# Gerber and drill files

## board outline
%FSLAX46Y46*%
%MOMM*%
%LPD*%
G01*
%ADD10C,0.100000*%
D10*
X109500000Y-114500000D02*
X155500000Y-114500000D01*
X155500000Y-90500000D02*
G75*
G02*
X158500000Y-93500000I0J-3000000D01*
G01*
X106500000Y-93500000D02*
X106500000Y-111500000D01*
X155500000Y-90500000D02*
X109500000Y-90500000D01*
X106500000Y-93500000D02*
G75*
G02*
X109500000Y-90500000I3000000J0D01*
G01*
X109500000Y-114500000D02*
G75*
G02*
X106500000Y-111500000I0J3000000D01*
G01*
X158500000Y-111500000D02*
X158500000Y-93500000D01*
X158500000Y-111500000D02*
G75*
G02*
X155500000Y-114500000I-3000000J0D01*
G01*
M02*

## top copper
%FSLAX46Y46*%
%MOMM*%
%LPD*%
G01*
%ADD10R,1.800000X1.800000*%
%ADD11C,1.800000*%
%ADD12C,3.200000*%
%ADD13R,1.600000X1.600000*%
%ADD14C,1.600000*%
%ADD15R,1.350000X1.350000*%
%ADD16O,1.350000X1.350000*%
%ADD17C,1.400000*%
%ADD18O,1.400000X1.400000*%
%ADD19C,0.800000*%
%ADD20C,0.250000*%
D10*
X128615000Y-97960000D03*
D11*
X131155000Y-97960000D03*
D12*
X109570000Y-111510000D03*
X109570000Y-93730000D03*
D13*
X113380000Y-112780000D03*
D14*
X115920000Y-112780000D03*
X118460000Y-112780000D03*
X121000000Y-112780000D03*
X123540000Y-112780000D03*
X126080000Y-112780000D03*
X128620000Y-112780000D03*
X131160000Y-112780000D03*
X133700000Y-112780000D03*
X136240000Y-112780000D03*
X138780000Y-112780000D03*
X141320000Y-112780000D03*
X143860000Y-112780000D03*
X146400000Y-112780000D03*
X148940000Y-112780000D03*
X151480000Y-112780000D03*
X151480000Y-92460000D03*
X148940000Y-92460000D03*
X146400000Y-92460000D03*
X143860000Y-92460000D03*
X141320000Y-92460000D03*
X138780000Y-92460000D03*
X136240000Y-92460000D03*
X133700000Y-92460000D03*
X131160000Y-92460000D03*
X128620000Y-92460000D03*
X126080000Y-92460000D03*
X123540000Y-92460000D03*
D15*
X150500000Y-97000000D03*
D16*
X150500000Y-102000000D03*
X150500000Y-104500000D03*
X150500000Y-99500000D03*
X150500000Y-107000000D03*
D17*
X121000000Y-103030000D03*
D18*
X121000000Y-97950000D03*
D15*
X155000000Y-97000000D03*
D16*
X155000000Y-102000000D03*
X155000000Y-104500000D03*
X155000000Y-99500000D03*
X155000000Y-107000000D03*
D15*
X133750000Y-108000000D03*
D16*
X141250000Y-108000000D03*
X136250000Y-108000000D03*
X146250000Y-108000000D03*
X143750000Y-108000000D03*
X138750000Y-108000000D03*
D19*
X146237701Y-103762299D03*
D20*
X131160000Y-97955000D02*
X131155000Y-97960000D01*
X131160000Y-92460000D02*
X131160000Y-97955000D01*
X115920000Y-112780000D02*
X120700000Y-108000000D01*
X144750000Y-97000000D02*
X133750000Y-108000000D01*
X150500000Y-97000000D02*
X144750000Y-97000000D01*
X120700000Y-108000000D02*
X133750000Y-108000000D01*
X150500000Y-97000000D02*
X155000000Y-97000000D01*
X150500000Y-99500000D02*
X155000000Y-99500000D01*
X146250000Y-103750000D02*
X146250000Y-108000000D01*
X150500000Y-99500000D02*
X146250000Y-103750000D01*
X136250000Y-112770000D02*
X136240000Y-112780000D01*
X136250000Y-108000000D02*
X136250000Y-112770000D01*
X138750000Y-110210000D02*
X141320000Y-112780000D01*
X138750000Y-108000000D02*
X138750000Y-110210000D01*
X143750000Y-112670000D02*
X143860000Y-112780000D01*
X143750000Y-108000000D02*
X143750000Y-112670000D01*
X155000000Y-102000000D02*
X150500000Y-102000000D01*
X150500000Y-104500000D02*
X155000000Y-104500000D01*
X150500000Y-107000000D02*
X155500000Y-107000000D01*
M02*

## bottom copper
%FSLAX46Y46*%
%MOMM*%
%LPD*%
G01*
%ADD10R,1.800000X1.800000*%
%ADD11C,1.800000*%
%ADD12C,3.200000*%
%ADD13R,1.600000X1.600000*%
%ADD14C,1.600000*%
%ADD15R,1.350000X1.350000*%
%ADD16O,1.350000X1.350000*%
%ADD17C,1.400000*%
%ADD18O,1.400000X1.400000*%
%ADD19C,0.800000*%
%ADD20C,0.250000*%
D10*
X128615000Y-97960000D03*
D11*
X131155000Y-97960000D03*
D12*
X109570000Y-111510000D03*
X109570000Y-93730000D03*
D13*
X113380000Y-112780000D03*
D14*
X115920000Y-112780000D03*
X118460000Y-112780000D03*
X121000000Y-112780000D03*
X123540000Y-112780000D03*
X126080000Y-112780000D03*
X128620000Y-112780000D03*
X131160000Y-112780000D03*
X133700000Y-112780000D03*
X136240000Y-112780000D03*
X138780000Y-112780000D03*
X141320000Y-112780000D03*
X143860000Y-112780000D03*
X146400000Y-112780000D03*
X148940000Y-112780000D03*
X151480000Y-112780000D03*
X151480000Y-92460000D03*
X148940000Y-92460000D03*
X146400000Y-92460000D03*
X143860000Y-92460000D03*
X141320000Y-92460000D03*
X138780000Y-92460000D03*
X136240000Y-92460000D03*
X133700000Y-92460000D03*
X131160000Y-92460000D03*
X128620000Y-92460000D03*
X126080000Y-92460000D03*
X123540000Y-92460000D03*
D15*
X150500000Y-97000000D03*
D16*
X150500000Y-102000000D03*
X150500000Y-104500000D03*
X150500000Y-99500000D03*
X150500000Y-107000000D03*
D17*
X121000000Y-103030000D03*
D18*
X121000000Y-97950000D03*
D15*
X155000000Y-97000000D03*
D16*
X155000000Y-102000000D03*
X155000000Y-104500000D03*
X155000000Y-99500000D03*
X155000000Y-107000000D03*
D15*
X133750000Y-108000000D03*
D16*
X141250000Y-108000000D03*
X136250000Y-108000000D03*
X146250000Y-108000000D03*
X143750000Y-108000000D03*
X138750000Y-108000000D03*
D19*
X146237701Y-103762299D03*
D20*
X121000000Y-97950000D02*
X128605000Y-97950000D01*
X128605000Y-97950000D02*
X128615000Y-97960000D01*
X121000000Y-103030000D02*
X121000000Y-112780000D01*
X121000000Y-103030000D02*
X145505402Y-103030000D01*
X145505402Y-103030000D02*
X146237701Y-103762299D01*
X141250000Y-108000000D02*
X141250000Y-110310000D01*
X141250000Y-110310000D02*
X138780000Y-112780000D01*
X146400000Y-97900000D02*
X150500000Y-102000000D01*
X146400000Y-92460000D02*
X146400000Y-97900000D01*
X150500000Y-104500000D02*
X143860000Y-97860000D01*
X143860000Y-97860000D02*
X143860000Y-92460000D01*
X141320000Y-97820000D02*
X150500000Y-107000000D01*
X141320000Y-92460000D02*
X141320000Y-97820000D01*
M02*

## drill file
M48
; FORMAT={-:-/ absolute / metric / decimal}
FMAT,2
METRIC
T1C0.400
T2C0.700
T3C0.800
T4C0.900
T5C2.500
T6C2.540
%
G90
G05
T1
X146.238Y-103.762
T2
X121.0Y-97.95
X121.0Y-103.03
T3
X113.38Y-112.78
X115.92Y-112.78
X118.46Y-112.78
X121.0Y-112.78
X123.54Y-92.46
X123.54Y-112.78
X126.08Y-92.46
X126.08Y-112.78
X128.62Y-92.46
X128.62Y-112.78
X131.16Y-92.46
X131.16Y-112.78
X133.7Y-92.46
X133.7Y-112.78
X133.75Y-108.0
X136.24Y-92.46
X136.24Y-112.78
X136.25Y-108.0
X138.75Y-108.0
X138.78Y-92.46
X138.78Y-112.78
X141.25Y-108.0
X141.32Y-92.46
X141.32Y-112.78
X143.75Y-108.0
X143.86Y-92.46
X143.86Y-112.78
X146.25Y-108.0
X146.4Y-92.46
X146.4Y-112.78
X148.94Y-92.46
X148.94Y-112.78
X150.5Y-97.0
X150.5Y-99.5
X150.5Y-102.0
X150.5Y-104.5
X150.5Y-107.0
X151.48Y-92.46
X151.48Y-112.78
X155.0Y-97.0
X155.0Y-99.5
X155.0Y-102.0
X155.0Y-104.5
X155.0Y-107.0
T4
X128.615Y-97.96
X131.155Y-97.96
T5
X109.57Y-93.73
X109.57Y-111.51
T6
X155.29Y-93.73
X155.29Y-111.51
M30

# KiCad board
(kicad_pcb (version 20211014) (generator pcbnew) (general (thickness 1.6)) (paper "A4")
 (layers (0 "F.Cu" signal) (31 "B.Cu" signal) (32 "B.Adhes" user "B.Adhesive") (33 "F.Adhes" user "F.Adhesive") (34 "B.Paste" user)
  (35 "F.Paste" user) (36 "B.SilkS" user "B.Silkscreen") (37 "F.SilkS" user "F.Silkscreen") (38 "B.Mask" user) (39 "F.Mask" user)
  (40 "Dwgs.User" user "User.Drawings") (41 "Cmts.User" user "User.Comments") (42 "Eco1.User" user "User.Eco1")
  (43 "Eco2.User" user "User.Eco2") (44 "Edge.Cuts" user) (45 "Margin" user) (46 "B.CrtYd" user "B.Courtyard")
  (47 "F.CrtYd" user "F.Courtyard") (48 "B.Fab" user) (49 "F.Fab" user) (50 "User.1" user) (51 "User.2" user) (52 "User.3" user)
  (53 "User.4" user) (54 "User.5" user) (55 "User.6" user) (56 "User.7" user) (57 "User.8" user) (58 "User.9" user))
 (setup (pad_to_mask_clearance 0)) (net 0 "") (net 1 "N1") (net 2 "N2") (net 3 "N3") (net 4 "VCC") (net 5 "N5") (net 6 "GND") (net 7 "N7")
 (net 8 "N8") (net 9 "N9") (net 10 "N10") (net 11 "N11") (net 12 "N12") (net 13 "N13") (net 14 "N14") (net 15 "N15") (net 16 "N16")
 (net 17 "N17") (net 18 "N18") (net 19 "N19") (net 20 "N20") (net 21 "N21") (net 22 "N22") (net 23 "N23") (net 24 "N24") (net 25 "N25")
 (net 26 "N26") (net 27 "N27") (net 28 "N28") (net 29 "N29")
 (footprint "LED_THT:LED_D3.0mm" (layer "F.Cu") (at 128.615 97.96)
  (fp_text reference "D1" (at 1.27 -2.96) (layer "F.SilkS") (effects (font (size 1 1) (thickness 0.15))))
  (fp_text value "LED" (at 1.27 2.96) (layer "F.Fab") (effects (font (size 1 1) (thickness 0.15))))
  (pad "1" thru_hole rect (at 0 0) (size 1.8 1.8) (drill 0.9) (layers *.Cu *.Mask) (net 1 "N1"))
  (pad "2" thru_hole circle (at 2.54 0) (size 1.8 1.8) (drill 0.9) (layers *.Cu *.Mask) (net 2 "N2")))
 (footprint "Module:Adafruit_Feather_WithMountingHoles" (layer "F.Cu") (at 113.38 112.78 90)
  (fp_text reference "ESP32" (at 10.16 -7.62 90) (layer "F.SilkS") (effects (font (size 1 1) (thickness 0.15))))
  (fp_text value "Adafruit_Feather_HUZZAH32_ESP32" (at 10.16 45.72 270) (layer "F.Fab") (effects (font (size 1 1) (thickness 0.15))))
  (pad "" np_thru_hole circle (at 1.27 -3.81) (size 3.2 3.2) (drill 2.5) (layers *.Cu *.Mask))
  (pad "" np_thru_hole circle (at 1.27 41.91) (size 2.54 2.54) (drill 2.54) (layers *.Cu *.Mask))
  (pad "" np_thru_hole circle (at 19.05 -3.81) (size 3.2 3.2) (drill 2.5) (layers *.Cu *.Mask))
  (pad "" np_thru_hole circle (at 19.05 41.91) (size 2.54 2.54) (drill 2.54) (layers *.Cu *.Mask))
  (pad "1" thru_hole rect (at 0 0 270) (size 1.6 1.6) (drill 0.8) (layers *.Cu *.Mask) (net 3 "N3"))
  (pad "2" thru_hole circle (at 0 2.54 270) (size 1.6 1.6) (drill 0.8) (layers *.Cu *.Mask) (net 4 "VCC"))
  (pad "3" thru_hole circle (at 0 5.08 270) (size 1.6 1.6) (drill 0.8) (layers *.Cu *.Mask) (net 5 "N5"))
  (pad "4" thru_hole circle (at 0 7.62 270) (size 1.6 1.6) (drill 0.8) (layers *.Cu *.Mask) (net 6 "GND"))
  (pad "5" thru_hole circle (at 0 10.16 270) (size 1.6 1.6) (drill 0.8) (layers *.Cu *.Mask) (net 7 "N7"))
  (pad "6" thru_hole circle (at 0 12.7 270) (size 1.6 1.6) (drill 0.8) (layers *.Cu *.Mask) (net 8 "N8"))
  (pad "7" thru_hole circle (at 0 15.24 270) (size 1.6 1.6) (drill 0.8) (layers *.Cu *.Mask) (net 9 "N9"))
  (pad "8" thru_hole circle (at 0 17.78 270) (size 1.6 1.6) (drill 0.8) (layers *.Cu *.Mask) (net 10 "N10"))
  (pad "9" thru_hole circle (at 0 20.32 270) (size 1.6 1.6) (drill 0.8) (layers *.Cu *.Mask) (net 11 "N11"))
  (pad "10" thru_hole circle (at 0 22.86 270) (size 1.6 1.6) (drill 0.8) (layers *.Cu *.Mask) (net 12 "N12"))
  (pad "11" thru_hole circle (at 0 25.4 270) (size 1.6 1.6) (drill 0.8) (layers *.Cu *.Mask) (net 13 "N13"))
  (pad "12" thru_hole circle (at 0 27.94 270) (size 1.6 1.6) (drill 0.8) (layers *.Cu *.Mask) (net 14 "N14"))
  (pad "13" thru_hole circle (at 0 30.48 270) (size 1.6 1.6) (drill 0.8) (layers *.Cu *.Mask) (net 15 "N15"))
  (pad "14" thru_hole circle (at 0 33.02 270) (size 1.6 1.6) (drill 0.8) (layers *.Cu *.Mask) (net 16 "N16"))
  (pad "15" thru_hole circle (at 0 35.56 270) (size 1.6 1.6) (drill 0.8) (layers *.Cu *.Mask) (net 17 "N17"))
  (pad "16" thru_hole circle (at 0 38.1 270) (size 1.6 1.6) (drill 0.8) (layers *.Cu *.Mask) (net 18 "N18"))
  (pad "17" thru_hole circle (at 20.32 38.1 270) (size 1.6 1.6) (drill 0.8) (layers *.Cu *.Mask) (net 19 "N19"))
  (pad "18" thru_hole circle (at 20.32 35.56 270) (size 1.6 1.6) (drill 0.8) (layers *.Cu *.Mask) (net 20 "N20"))
  (pad "19" thru_hole circle (at 20.32 33.02 270) (size 1.6 1.6) (drill 0.8) (layers *.Cu *.Mask) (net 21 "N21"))
  (pad "20" thru_hole circle (at 20.32 30.48 270) (size 1.6 1.6) (drill 0.8) (layers *.Cu *.Mask) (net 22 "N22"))
  (pad "21" thru_hole circle (at 20.32 27.94 270) (size 1.6 1.6) (drill 0.8) (layers *.Cu *.Mask) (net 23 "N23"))
  (pad "22" thru_hole circle (at 20.32 25.4 270) (size 1.6 1.6) (drill 0.8) (layers *.Cu *.Mask) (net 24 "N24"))
  (pad "23" thru_hole circle (at 20.32 22.86 270) (size 1.6 1.6) (drill 0.8) (layers *.Cu *.Mask) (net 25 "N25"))
  (pad "24" thru_hole circle (at 20.32 20.32 270) (size 1.6 1.6) (drill 0.8) (layers *.Cu *.Mask) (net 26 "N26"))
  (pad "25" thru_hole circle (at 20.32 17.78 270) (size 1.6 1.6) (drill 0.8) (layers *.Cu *.Mask) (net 2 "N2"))
  (pad "26" thru_hole circle (at 20.32 15.24 270) (size 1.6 1.6) (drill 0.8) (layers *.Cu *.Mask) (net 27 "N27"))
  (pad "27" thru_hole circle (at 20.32 12.7 270) (size 1.6 1.6) (drill 0.8) (layers *.Cu *.Mask) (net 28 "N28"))
  (pad "28" thru_hole circle (at 20.32 10.16 270) (size 1.6 1.6) (drill 0.8) (layers *.Cu *.Mask) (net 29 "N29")))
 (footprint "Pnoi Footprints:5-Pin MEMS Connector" (layer "F.Cu") (at 150.5 107 180)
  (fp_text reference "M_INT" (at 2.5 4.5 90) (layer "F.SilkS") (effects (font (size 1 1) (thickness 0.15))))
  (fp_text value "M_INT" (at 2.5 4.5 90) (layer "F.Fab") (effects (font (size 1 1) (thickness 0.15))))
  (pad "3V" thru_hole rect (at 0 10 90) (size 1.35 1.35) (drill 0.8) (layers *.Cu *.Mask) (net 4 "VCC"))
  (pad "BCLK" thru_hole oval (at 0 5) (size 1.35 1.35) (drill 0.8) (layers *.Cu *.Mask) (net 21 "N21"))
  (pad "DOUT" thru_hole oval (at 0 2.5) (size 1.35 1.35) (drill 0.8) (layers *.Cu *.Mask) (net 22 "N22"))
  (pad "GND" thru_hole oval (at 0 7.5) (size 1.35 1.35) (drill 0.8) (layers *.Cu *.Mask) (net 6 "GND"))
  (pad "LRCL" thru_hole oval (at 0 0) (size 1.35 1.35) (drill 0.8) (layers *.Cu *.Mask) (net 23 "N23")))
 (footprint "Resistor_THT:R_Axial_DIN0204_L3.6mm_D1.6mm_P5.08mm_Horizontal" (layer "F.Cu") (at 121 103.03 90)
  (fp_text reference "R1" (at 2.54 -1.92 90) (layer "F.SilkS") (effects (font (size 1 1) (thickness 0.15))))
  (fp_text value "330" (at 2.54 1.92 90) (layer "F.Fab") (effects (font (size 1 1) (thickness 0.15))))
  (pad "1" thru_hole circle (at 0 0 90) (size 1.4 1.4) (drill 0.7) (layers *.Cu *.Mask) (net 6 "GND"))
  (pad "2" thru_hole oval (at 5.08 0 90) (size 1.4 1.4) (drill 0.7) (layers *.Cu *.Mask) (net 1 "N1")))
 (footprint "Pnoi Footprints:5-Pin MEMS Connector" (layer "F.Cu") (at 155 107 180)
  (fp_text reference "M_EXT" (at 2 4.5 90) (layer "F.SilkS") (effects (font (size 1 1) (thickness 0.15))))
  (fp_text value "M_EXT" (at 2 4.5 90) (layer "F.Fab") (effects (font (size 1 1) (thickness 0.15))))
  (pad "3V" thru_hole rect (at 0 10 90) (size 1.35 1.35) (drill 0.8) (layers *.Cu *.Mask) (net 4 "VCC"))
  (pad "BCLK" thru_hole oval (at 0 5) (size 1.35 1.35) (drill 0.8) (layers *.Cu *.Mask) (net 21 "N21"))
  (pad "DOUT" thru_hole oval (at 0 2.5) (size 1.35 1.35) (drill 0.8) (layers *.Cu *.Mask) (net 22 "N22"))
  (pad "GND" thru_hole oval (at 0 7.5) (size 1.35 1.35) (drill 0.8) (layers *.Cu *.Mask) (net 6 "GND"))
  (pad "LRCL" thru_hole oval (at 0 0) (size 1.35 1.35) (drill 0.8) (layers *.Cu *.Mask) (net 23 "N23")))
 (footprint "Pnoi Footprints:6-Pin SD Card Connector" (layer "F.Cu") (at 133.75 108 90)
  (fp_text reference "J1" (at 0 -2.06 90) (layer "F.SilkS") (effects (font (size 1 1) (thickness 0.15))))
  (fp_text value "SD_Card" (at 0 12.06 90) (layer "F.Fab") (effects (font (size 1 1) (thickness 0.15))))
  (pad "3v3" thru_hole rect (at 0 0 90) (size 1.35 1.35) (drill 0.8) (layers *.Cu *.Mask) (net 4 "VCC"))
  (pad "CLK" thru_hole oval (at 0 7.5 90) (size 1.35 1.35) (drill 0.8) (layers *.Cu *.Mask) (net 13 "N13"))
  (pad "CS" thru_hole oval (at 0 2.5 90) (size 1.35 1.35) (drill 0.8) (layers *.Cu *.Mask) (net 12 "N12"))
  (pad "GND" thru_hole oval (at 0 12.5 90) (size 1.35 1.35) (drill 0.8) (layers *.Cu *.Mask) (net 6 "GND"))
  (pad "MISO" thru_hole oval (at 0 10 90) (size 1.35 1.35) (drill 0.8) (layers *.Cu *.Mask) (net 15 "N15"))
  (pad "MOSI" thru_hole oval (at 0 5 90) (size 1.35 1.35) (drill 0.8) (layers *.Cu *.Mask) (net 14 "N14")))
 (gr_line (start 109.5 114.5) (end 155.5 114.5) (layer "Edge.Cuts") (width 0.1))
 (gr_arc (start 155.5 90.5) (mid 157.62132 91.37868) (end 158.5 93.5) (layer "Edge.Cuts") (width 0.1))
 (gr_line (start 106.5 93.5) (end 106.5 111.5) (layer "Edge.Cuts") (width 0.1))
 (gr_line (start 155.5 90.5) (end 109.5 90.5) (layer "Edge.Cuts") (width 0.1))
 (gr_arc (start 106.5 93.5) (mid 107.37868 91.37868) (end 109.5 90.5) (layer "Edge.Cuts") (width 0.1))
 (gr_arc (start 109.5 114.5) (mid 107.37868 113.62132) (end 106.5 111.5) (layer "Edge.Cuts") (width 0.1))
 (gr_line (start 158.5 111.5) (end 158.5 93.5) (layer "Edge.Cuts") (width 0.1))
 (gr_arc (start 158.5 111.5) (mid 157.62132 113.62132) (end 155.5 114.5) (layer "Edge.Cuts") (width 0.1))
 (segment (start 121 97.95) (end 128.605 97.95) (width 0.25) (layer "B.Cu") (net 1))
 (segment (start 128.605 97.95) (end 128.615 97.96) (width 0.25) (layer "B.Cu") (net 1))
 (segment (start 131.16 97.955) (end 131.155 97.96) (width 0.25) (layer "F.Cu") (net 2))
 (segment (start 131.16 92.46) (end 131.16 97.955) (width 0.25) (layer "F.Cu") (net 2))
 (segment (start 115.92 112.78) (end 120.7 108) (width 0.25) (layer "F.Cu") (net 4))
 (segment (start 144.75 97) (end 133.75 108) (width 0.25) (layer "F.Cu") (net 4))
 (segment (start 150.5 97) (end 144.75 97) (width 0.25) (layer "F.Cu") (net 4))
 (segment (start 120.7 108) (end 133.75 108) (width 0.25) (layer "F.Cu") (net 4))
 (segment (start 150.5 97) (end 155 97) (width 0.25) (layer "F.Cu") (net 4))
 (segment (start 150.5 99.5) (end 155 99.5) (width 0.25) (layer "F.Cu") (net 6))
 (segment (start 146.25 103.75) (end 146.25 108) (width 0.25) (layer "F.Cu") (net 6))
 (segment (start 150.5 99.5) (end 146.25 103.75) (width 0.25) (layer "F.Cu") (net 6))
 (via (at 146.237701 103.762299) (size 0.8) (drill 0.4) (layers "F.Cu" "B.Cu") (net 6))
 (segment (start 121 103.03) (end 121 112.78) (width 0.25) (layer "B.Cu") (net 6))
 (segment (start 121 103.03) (end 145.505402 103.03) (width 0.25) (layer "B.Cu") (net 6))
 (segment (start 145.505402 103.03) (end 146.237701 103.762299) (width 0.25) (layer "B.Cu") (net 6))
 (segment (start 136.25 112.77) (end 136.24 112.78) (width 0.25) (layer "F.Cu") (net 12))
 (segment (start 136.25 108) (end 136.25 112.77) (width 0.25) (layer "F.Cu") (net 12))
 (segment (start 141.25 108) (end 141.25 110.31) (width 0.25) (layer "B.Cu") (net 13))
 (segment (start 141.25 110.31) (end 138.78 112.78) (width 0.25) (layer "B.Cu") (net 13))
 (segment (start 138.75 110.21) (end 141.32 112.78) (width 0.25) (layer "F.Cu") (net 14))
 (segment (start 138.75 108) (end 138.75 110.21) (width 0.25) (layer "F.Cu") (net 14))
 (segment (start 143.75 112.67) (end 143.86 112.78) (width 0.25) (layer "F.Cu") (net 15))
 (segment (start 143.75 108) (end 143.75 112.67) (width 0.25) (layer "F.Cu") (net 15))
 (segment (start 155 102) (end 150.5 102) (width 0.25) (layer "F.Cu") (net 21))
 (segment (start 146.4 97.9) (end 150.5 102) (width 0.25) (layer "B.Cu") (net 21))
 (segment (start 146.4 92.46) (end 146.4 97.9) (width 0.25) (layer "B.Cu") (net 21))
 (segment (start 150.5 104.5) (end 155 104.5) (width 0.25) (layer "F.Cu") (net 22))
 (segment (start 150.5 104.5) (end 143.86 97.86) (width 0.25) (layer "B.Cu") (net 22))
 (segment (start 143.86 97.86) (end 143.86 92.46) (width 0.25) (layer "B.Cu") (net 22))
 (segment (start 150.5 107) (end 155.5 107) (width 0.25) (layer "F.Cu") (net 23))
 (segment (start 141.32 97.82) (end 150.5 107) (width 0.25) (layer "B.Cu") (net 23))
 (segment (start 141.32 92.46) (end 141.32 97.82) (width 0.25) (layer "B.Cu") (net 23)))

